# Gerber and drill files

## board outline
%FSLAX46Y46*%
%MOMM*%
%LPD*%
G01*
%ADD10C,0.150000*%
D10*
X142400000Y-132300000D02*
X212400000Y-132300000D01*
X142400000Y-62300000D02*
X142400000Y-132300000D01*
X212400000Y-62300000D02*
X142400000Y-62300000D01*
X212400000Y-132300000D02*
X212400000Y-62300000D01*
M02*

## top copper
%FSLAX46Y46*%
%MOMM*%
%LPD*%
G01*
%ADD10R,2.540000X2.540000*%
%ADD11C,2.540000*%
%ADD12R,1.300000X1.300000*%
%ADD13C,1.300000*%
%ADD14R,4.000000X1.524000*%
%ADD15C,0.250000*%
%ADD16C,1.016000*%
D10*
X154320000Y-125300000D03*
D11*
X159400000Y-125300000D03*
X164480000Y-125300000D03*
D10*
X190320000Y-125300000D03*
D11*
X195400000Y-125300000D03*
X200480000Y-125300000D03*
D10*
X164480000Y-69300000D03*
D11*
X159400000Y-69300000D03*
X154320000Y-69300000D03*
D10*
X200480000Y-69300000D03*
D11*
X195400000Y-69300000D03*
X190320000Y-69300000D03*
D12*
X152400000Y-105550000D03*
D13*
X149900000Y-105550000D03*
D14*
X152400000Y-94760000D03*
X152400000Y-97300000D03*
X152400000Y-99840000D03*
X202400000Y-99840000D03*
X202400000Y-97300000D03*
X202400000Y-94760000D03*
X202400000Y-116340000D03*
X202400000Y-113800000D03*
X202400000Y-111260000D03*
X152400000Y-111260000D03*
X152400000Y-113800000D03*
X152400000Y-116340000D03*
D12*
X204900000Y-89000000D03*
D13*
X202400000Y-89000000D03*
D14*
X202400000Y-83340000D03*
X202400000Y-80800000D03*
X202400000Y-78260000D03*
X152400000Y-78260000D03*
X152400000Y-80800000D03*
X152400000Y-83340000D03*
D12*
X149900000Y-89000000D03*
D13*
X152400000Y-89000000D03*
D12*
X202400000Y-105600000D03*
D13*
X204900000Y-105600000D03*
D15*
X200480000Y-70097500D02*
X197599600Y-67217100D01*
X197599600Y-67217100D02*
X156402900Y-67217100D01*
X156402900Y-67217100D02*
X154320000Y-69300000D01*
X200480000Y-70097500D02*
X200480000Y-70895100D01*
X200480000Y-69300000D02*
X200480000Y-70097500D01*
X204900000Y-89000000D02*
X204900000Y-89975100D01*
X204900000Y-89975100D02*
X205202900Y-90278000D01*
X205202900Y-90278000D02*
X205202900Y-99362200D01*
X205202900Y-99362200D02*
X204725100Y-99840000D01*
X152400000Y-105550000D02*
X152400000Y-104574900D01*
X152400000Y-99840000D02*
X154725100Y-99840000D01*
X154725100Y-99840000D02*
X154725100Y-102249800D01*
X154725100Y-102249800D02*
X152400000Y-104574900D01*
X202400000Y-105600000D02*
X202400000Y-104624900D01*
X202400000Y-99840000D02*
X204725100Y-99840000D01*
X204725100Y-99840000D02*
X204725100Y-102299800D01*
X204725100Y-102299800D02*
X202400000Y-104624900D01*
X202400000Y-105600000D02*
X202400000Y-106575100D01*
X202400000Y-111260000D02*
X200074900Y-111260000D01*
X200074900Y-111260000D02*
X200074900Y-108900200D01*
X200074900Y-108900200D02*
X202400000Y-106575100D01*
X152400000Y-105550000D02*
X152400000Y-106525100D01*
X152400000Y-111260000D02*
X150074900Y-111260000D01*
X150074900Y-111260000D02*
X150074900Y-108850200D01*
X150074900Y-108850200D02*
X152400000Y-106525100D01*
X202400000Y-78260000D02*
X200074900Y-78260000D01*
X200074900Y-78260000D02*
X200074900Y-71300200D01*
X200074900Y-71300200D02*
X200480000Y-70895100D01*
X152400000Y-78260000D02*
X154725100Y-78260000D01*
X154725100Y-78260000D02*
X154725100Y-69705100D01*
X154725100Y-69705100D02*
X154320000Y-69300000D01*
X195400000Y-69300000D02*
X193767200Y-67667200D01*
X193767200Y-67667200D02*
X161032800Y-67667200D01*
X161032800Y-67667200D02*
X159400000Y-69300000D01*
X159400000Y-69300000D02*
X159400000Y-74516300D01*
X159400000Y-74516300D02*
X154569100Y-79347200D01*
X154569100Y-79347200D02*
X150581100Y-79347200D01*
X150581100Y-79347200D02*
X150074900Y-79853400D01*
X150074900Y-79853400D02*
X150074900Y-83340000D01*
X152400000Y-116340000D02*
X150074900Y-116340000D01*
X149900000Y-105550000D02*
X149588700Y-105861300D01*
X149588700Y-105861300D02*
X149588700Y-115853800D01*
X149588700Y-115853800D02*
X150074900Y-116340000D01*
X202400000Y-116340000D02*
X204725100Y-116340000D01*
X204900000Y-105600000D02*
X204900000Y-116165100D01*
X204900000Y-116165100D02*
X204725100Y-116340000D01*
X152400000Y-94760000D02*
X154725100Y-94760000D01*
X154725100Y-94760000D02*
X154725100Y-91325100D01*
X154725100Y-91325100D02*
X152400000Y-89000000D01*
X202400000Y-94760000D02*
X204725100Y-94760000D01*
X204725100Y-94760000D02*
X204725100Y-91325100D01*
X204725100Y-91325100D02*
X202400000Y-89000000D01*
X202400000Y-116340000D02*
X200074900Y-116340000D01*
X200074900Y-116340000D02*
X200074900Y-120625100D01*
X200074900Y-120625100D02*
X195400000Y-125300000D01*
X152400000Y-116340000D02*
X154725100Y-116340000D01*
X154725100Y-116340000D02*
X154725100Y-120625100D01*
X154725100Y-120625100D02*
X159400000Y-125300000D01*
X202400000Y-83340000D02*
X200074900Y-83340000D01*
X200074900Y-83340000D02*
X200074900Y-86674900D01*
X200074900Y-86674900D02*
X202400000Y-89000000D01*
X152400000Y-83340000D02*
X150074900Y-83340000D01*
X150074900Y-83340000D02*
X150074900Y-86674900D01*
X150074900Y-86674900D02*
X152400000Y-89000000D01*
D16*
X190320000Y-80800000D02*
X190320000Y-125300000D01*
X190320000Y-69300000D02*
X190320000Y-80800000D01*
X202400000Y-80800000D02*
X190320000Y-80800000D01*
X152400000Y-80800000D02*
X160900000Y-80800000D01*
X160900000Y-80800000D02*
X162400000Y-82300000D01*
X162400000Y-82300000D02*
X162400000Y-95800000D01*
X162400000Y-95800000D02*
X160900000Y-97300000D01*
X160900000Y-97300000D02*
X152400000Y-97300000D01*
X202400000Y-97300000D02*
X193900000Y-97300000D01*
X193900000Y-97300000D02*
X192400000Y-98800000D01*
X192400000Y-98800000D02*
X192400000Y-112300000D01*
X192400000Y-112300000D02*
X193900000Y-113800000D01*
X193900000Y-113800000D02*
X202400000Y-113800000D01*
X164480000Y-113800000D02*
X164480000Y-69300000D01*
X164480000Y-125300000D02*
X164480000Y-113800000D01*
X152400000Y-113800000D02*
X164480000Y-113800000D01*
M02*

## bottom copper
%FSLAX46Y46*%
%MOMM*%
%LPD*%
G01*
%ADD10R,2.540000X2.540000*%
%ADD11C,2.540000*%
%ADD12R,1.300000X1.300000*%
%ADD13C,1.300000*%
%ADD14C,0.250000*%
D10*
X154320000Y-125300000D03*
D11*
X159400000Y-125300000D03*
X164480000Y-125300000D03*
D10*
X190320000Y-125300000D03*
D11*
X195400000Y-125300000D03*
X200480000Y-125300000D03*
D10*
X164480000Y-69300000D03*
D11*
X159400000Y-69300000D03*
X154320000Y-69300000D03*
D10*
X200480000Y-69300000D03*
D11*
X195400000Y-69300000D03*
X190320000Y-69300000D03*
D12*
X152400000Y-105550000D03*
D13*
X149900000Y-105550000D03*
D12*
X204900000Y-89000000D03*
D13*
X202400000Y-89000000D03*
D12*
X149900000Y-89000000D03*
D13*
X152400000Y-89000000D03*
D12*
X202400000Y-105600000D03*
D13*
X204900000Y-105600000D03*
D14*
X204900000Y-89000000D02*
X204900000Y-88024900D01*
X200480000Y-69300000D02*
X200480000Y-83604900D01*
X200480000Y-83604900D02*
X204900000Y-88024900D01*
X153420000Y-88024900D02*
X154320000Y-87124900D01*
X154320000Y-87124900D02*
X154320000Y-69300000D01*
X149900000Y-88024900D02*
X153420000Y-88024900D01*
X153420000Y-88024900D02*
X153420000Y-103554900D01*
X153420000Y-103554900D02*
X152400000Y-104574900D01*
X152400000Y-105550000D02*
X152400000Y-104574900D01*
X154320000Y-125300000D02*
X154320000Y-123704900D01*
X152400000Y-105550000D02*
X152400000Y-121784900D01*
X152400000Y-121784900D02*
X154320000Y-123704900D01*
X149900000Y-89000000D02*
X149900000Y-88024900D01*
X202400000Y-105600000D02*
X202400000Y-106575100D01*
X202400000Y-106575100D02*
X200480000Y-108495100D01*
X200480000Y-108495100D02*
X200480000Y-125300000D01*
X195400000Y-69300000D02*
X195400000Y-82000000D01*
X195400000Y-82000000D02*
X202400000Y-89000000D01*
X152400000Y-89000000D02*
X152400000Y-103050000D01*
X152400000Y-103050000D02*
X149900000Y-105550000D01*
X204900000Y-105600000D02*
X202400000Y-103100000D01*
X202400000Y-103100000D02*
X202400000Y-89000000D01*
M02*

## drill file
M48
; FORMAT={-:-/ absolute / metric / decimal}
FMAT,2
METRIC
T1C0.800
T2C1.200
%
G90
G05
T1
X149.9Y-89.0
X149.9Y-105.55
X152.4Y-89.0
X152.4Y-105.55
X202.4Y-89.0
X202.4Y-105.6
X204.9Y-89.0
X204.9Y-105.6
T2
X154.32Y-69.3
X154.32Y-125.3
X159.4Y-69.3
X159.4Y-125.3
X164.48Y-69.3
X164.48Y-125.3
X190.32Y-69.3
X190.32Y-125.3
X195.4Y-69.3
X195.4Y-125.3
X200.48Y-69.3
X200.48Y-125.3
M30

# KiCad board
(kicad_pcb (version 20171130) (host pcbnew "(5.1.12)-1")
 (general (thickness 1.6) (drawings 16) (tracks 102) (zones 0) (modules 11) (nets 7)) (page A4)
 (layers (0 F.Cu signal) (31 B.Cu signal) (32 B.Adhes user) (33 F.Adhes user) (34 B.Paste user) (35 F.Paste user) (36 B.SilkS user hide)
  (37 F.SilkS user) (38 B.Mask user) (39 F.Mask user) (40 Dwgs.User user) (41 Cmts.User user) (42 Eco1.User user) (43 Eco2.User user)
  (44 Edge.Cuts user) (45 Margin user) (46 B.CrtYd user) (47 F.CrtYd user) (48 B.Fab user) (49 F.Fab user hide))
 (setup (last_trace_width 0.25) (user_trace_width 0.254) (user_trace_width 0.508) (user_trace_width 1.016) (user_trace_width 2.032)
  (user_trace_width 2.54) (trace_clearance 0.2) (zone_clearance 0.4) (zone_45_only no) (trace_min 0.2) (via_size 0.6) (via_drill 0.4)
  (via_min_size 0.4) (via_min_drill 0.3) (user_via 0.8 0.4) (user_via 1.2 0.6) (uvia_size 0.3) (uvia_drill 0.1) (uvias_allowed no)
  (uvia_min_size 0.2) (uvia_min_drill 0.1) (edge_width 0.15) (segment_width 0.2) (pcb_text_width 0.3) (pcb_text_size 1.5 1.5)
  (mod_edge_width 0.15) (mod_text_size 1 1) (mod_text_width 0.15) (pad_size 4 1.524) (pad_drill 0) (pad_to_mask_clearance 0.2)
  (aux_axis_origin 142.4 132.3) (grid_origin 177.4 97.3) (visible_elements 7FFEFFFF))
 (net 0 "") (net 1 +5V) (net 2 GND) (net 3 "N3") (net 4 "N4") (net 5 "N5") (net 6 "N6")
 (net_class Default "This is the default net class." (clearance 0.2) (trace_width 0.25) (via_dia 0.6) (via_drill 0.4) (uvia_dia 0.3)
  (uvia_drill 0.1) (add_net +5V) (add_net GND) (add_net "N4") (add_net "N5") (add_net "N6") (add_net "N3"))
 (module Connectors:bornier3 (layer F.Cu) (at 159.4 125.3)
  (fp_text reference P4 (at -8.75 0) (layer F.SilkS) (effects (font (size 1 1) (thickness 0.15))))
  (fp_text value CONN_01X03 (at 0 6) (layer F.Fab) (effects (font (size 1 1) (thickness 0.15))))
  (pad 1 thru_hole rect (at -5.08 0) (size 2.54 2.54) (drill 1.2) (layers *.Cu *.Mask) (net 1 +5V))
  (pad 2 thru_hole circle (at 0 0) (size 2.54 2.54) (drill 1.2) (layers *.Cu *.Mask) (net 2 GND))
  (pad 3 thru_hole circle (at 5.08 0) (size 2.54 2.54) (drill 1.2) (layers *.Cu *.Mask) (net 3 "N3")))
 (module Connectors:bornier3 (layer F.Cu) (at 195.4 125.3)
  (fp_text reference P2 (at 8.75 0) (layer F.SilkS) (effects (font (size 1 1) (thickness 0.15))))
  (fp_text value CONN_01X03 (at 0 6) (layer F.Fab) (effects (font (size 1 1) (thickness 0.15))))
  (pad 1 thru_hole rect (at -5.08 0) (size 2.54 2.54) (drill 1.2) (layers *.Cu *.Mask) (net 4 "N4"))
  (pad 2 thru_hole circle (at 0 0) (size 2.54 2.54) (drill 1.2) (layers *.Cu *.Mask) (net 2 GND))
  (pad 3 thru_hole circle (at 5.08 0) (size 2.54 2.54) (drill 1.2) (layers *.Cu *.Mask) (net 1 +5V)))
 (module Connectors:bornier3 (layer F.Cu) (at 159.4 69.3 180)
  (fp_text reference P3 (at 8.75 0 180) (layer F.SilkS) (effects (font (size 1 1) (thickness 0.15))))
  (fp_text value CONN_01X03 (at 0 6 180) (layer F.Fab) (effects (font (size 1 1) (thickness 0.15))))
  (pad 1 thru_hole rect (at -5.08 0 180) (size 2.54 2.54) (drill 1.2) (layers *.Cu *.Mask) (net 3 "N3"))
  (pad 2 thru_hole circle (at 0 0 180) (size 2.54 2.54) (drill 1.2) (layers *.Cu *.Mask) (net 2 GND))
  (pad 3 thru_hole circle (at 5.08 0 180) (size 2.54 2.54) (drill 1.2) (layers *.Cu *.Mask) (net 1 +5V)))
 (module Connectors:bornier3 (layer F.Cu) (at 195.4 69.3 180)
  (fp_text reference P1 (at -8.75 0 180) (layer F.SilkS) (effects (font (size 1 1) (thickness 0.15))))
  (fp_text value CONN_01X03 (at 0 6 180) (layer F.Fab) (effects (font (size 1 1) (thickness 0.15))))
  (pad 1 thru_hole rect (at -5.08 0 180) (size 2.54 2.54) (drill 1.2) (layers *.Cu *.Mask) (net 1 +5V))
  (pad 2 thru_hole circle (at 0 0 180) (size 2.54 2.54) (drill 1.2) (layers *.Cu *.Mask) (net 2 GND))
  (pad 3 thru_hole circle (at 5.08 0 180) (size 2.54 2.54) (drill 1.2) (layers *.Cu *.Mask) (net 4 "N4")))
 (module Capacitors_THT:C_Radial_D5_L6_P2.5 (layer F.Cu) (at 152.4 105.55 180)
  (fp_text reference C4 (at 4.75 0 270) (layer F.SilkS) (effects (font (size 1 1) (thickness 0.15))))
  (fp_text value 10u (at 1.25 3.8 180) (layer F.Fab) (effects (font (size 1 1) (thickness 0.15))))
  (pad 1 thru_hole rect (at 0 0 180) (size 1.3 1.3) (drill 0.8) (layers *.Cu *.Mask) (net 1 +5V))
  (pad 2 thru_hole circle (at 2.5 0 180) (size 1.3 1.3) (drill 0.8) (layers *.Cu *.Mask) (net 2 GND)))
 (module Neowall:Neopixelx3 (layer F.Cu) (at 152.4 97.3)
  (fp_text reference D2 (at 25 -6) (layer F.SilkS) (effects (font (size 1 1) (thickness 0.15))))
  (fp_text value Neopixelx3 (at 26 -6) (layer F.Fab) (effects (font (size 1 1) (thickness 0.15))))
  (pad 1 smd rect (at 0 -2.54) (size 4 1.524) (layers F.Cu F.Paste F.Mask) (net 2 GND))
  (pad 2 smd rect (at 0 0) (size 4 1.524) (layers F.Cu F.Paste F.Mask) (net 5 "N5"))
  (pad 3 smd rect (at 0 2.54) (size 4 1.524) (layers F.Cu F.Paste F.Mask) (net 1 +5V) (thermal_width 0.5) (thermal_gap 0.8))
  (pad 4 smd rect (at 50 2.54) (size 4 1.524) (layers F.Cu F.Paste F.Mask) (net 1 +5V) (thermal_gap 0.8))
  (pad 5 smd rect (at 50 0) (size 4 1.524) (layers F.Cu F.Paste F.Mask) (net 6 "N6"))
  (pad 6 smd rect (at 50 -2.54) (size 4 1.524) (layers F.Cu F.Paste F.Mask) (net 2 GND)))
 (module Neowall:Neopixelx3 (layer F.Cu) (at 202.4 113.8 180)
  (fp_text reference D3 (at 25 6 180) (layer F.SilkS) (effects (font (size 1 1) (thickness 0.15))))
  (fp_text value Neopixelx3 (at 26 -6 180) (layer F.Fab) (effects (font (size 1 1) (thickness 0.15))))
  (pad 1 smd rect (at 0 -2.54 180) (size 4 1.524) (layers F.Cu F.Paste F.Mask) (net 2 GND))
  (pad 2 smd rect (at 0 0 180) (size 4 1.524) (layers F.Cu F.Paste F.Mask) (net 6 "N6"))
  (pad 3 smd rect (at 0 2.54 180) (size 4 1.524) (layers F.Cu F.Paste F.Mask) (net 1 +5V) (thermal_width 0.5) (thermal_gap 0.8))
  (pad 4 smd rect (at 50 2.54 180) (size 4 1.524) (layers F.Cu F.Paste F.Mask) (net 1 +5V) (thermal_width 0.5) (thermal_gap 0.8))
  (pad 5 smd rect (at 50 0 180) (size 4 1.524) (layers F.Cu F.Paste F.Mask) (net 3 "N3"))
  (pad 6 smd rect (at 50 -2.54 180) (size 4 1.524) (layers F.Cu F.Paste F.Mask) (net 2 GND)))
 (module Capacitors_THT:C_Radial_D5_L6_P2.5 (layer F.Cu) (at 204.9 89 180)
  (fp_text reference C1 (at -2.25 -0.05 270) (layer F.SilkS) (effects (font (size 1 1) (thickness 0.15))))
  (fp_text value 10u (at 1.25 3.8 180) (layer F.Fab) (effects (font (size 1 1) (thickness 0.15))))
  (pad 1 thru_hole rect (at 0 0 180) (size 1.3 1.3) (drill 0.8) (layers *.Cu *.Mask) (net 1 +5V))
  (pad 2 thru_hole circle (at 2.5 0 180) (size 1.3 1.3) (drill 0.8) (layers *.Cu *.Mask) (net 2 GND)))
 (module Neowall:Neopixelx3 (layer F.Cu) (at 202.4 80.8 180)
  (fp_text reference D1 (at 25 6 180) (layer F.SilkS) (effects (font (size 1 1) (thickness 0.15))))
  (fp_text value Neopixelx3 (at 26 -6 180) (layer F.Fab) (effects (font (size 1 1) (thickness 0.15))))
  (pad 1 smd rect (at 0 -2.54 180) (size 4 1.524) (layers F.Cu F.Paste F.Mask) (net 2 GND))
  (pad 2 smd rect (at 0 0 180) (size 4 1.524) (layers F.Cu F.Paste F.Mask) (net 4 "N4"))
  (pad 3 smd rect (at 0 2.54 180) (size 4 1.524) (layers F.Cu F.Paste F.Mask) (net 1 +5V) (thermal_width 0.5) (thermal_gap 0.8))
  (pad 4 smd rect (at 50 2.54 180) (size 4 1.524) (layers F.Cu F.Paste F.Mask) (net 1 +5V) (thermal_width 0.5) (thermal_gap 0.8))
  (pad 5 smd rect (at 50 0 180) (size 4 1.524) (layers F.Cu F.Paste F.Mask) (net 5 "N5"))
  (pad 6 smd rect (at 50 -2.54 180) (size 4 1.524) (layers F.Cu F.Paste F.Mask) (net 2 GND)))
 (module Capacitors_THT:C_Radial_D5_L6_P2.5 (layer F.Cu) (at 149.9 89)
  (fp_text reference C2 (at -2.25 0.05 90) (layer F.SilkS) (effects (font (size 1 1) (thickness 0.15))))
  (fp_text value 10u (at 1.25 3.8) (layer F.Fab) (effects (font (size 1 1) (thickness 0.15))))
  (pad 1 thru_hole rect (at 0 0) (size 1.3 1.3) (drill 0.8) (layers *.Cu *.Mask) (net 1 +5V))
  (pad 2 thru_hole circle (at 2.5 0) (size 1.3 1.3) (drill 0.8) (layers *.Cu *.Mask) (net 2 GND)))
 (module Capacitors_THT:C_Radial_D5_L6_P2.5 (layer F.Cu) (at 202.4 105.6)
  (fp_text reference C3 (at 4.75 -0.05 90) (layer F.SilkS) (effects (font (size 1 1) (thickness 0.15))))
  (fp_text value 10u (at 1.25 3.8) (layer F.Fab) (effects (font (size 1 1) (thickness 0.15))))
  (pad 1 thru_hole rect (at 0 0) (size 1.3 1.3) (drill 0.8) (layers *.Cu *.Mask) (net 1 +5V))
  (pad 2 thru_hole circle (at 2.5 0) (size 1.3 1.3) (drill 0.8) (layers *.Cu *.Mask) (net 2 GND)))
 (gr_line (start 142.4 132.3) (end 212.4 132.3) (angle 90) (layer Edge.Cuts) (width 0.15))
 (gr_line (start 142.4 62.3) (end 142.4 132.3) (angle 90) (layer Edge.Cuts) (width 0.15))
 (gr_line (start 212.4 62.3) (end 142.4 62.3) (angle 90) (layer Edge.Cuts) (width 0.15))
 (gr_line (start 212.4 132.3) (end 212.4 62.3) (angle 90) (layer Edge.Cuts) (width 0.15))
 (segment (start 200.48 70.0975) (end 197.5996 67.2171) (width 0.25) (layer F.Cu) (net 1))
 (segment (start 197.5996 67.2171) (end 156.4029 67.2171) (width 0.25) (layer F.Cu) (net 1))
 (segment (start 156.4029 67.2171) (end 154.32 69.3) (width 0.25) (layer F.Cu) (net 1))
 (segment (start 200.48 70.0975) (end 200.48 70.8951) (width 0.25) (layer F.Cu) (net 1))
 (segment (start 200.48 69.3) (end 200.48 70.0975) (width 0.25) (layer F.Cu) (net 1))
 (segment (start 204.9 89) (end 204.9 88.0249) (width 0.25) (layer B.Cu) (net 1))
 (segment (start 200.48 69.3) (end 200.48 83.6049) (width 0.25) (layer B.Cu) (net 1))
 (segment (start 200.48 83.6049) (end 204.9 88.0249) (width 0.25) (layer B.Cu) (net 1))
 (segment (start 153.42 88.0249) (end 154.32 87.1249) (width 0.25) (layer B.Cu) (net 1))
 (segment (start 154.32 87.1249) (end 154.32 69.3) (width 0.25) (layer B.Cu) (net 1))
 (segment (start 149.9 88.0249) (end 153.42 88.0249) (width 0.25) (layer B.Cu) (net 1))
 (segment (start 153.42 88.0249) (end 153.42 103.5549) (width 0.25) (layer B.Cu) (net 1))
 (segment (start 153.42 103.5549) (end 152.4 104.5749) (width 0.25) (layer B.Cu) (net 1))
 (segment (start 152.4 105.55) (end 152.4 104.5749) (width 0.25) (layer B.Cu) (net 1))
 (segment (start 154.32 125.3) (end 154.32 123.7049) (width 0.25) (layer B.Cu) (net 1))
 (segment (start 152.4 105.55) (end 152.4 121.7849) (width 0.25) (layer B.Cu) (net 1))
 (segment (start 152.4 121.7849) (end 154.32 123.7049) (width 0.25) (layer B.Cu) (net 1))
 (segment (start 204.9 89) (end 204.9 89.9751) (width 0.25) (layer F.Cu) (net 1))
 (segment (start 204.9 89.9751) (end 205.2029 90.278) (width 0.25) (layer F.Cu) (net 1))
 (segment (start 205.2029 90.278) (end 205.2029 99.3622) (width 0.25) (layer F.Cu) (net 1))
 (segment (start 205.2029 99.3622) (end 204.7251 99.84) (width 0.25) (layer F.Cu) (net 1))
 (segment (start 149.9 89) (end 149.9 88.0249) (width 0.25) (layer B.Cu) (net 1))
 (segment (start 202.4 105.6) (end 202.4 106.5751) (width 0.25) (layer B.Cu) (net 1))
 (segment (start 202.4 106.5751) (end 200.48 108.4951) (width 0.25) (layer B.Cu) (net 1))
 (segment (start 200.48 108.4951) (end 200.48 125.3) (width 0.25) (layer B.Cu) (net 1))
 (segment (start 152.4 105.55) (end 152.4 104.5749) (width 0.25) (layer F.Cu) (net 1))
 (segment (start 152.4 99.84) (end 154.7251 99.84) (width 0.25) (layer F.Cu) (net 1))
 (segment (start 154.7251 99.84) (end 154.7251 102.2498) (width 0.25) (layer F.Cu) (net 1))
 (segment (start 154.7251 102.2498) (end 152.4 104.5749) (width 0.25) (layer F.Cu) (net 1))
 (segment (start 202.4 105.6) (end 202.4 104.6249) (width 0.25) (layer F.Cu) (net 1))
 (segment (start 202.4 99.84) (end 204.7251 99.84) (width 0.25) (layer F.Cu) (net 1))
 (segment (start 204.7251 99.84) (end 204.7251 102.2998) (width 0.25) (layer F.Cu) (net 1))
 (segment (start 204.7251 102.2998) (end 202.4 104.6249) (width 0.25) (layer F.Cu) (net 1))
 (segment (start 202.4 105.6) (end 202.4 106.5751) (width 0.25) (layer F.Cu) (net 1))
 (segment (start 202.4 111.26) (end 200.0749 111.26) (width 0.25) (layer F.Cu) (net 1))
 (segment (start 200.0749 111.26) (end 200.0749 108.9002) (width 0.25) (layer F.Cu) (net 1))
 (segment (start 200.0749 108.9002) (end 202.4 106.5751) (width 0.25) (layer F.Cu) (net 1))
 (segment (start 152.4 105.55) (end 152.4 106.5251) (width 0.25) (layer F.Cu) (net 1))
 (segment (start 152.4 111.26) (end 150.0749 111.26) (width 0.25) (layer F.Cu) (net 1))
 (segment (start 150.0749 111.26) (end 150.0749 108.8502) (width 0.25) (layer F.Cu) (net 1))
 (segment (start 150.0749 108.8502) (end 152.4 106.5251) (width 0.25) (layer F.Cu) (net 1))
 (segment (start 202.4 78.26) (end 200.0749 78.26) (width 0.25) (layer F.Cu) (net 1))
 (segment (start 200.0749 78.26) (end 200.0749 71.3002) (width 0.25) (layer F.Cu) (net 1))
 (segment (start 200.0749 71.3002) (end 200.48 70.8951) (width 0.25) (layer F.Cu) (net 1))
 (segment (start 152.4 78.26) (end 154.7251 78.26) (width 0.25) (layer F.Cu) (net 1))
 (segment (start 154.7251 78.26) (end 154.7251 69.7051) (width 0.25) (layer F.Cu) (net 1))
 (segment (start 154.7251 69.7051) (end 154.32 69.3) (width 0.25) (layer F.Cu) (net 1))
 (segment (start 195.4 69.3) (end 193.7672 67.6672) (width 0.25) (layer F.Cu) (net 2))
 (segment (start 193.7672 67.6672) (end 161.0328 67.6672) (width 0.25) (layer F.Cu) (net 2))
 (segment (start 161.0328 67.6672) (end 159.4 69.3) (width 0.25) (layer F.Cu) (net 2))
 (segment (start 195.4 69.3) (end 195.4 82) (width 0.25) (layer B.Cu) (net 2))
 (segment (start 195.4 82) (end 202.4 89) (width 0.25) (layer B.Cu) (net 2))
 (segment (start 159.4 69.3) (end 159.4 74.5163) (width 0.25) (layer F.Cu) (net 2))
 (segment (start 159.4 74.5163) (end 154.5691 79.3472) (width 0.25) (layer F.Cu) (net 2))
 (segment (start 154.5691 79.3472) (end 150.5811 79.3472) (width 0.25) (layer F.Cu) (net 2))
 (segment (start 150.5811 79.3472) (end 150.0749 79.8534) (width 0.25) (layer F.Cu) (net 2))
 (segment (start 150.0749 79.8534) (end 150.0749 83.34) (width 0.25) (layer F.Cu) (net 2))
 (segment (start 152.4 89) (end 152.4 103.05) (width 0.25) (layer B.Cu) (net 2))
 (segment (start 152.4 103.05) (end 149.9 105.55) (width 0.25) (layer B.Cu) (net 2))
 (segment (start 152.4 116.34) (end 150.0749 116.34) (width 0.25) (layer F.Cu) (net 2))
 (segment (start 149.9 105.55) (end 149.5887 105.8613) (width 0.25) (layer F.Cu) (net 2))
 (segment (start 149.5887 105.8613) (end 149.5887 115.8538) (width 0.25) (layer F.Cu) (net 2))
 (segment (start 149.5887 115.8538) (end 150.0749 116.34) (width 0.25) (layer F.Cu) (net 2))
 (segment (start 202.4 116.34) (end 204.7251 116.34) (width 0.25) (layer F.Cu) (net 2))
 (segment (start 204.9 105.6) (end 204.9 116.1651) (width 0.25) (layer F.Cu) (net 2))
 (segment (start 204.9 116.1651) (end 204.7251 116.34) (width 0.25) (layer F.Cu) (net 2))
 (segment (start 204.9 105.6) (end 202.4 103.1) (width 0.25) (layer B.Cu) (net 2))
 (segment (start 202.4 103.1) (end 202.4 89) (width 0.25) (layer B.Cu) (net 2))
 (segment (start 152.4 94.76) (end 154.7251 94.76) (width 0.25) (layer F.Cu) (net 2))
 (segment (start 154.7251 94.76) (end 154.7251 91.3251) (width 0.25) (layer F.Cu) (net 2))
 (segment (start 154.7251 91.3251) (end 152.4 89) (width 0.25) (layer F.Cu) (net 2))
 (segment (start 202.4 94.76) (end 204.7251 94.76) (width 0.25) (layer F.Cu) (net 2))
 (segment (start 204.7251 94.76) (end 204.7251 91.3251) (width 0.25) (layer F.Cu) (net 2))
 (segment (start 204.7251 91.3251) (end 202.4 89) (width 0.25) (layer F.Cu) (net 2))
 (segment (start 202.4 116.34) (end 200.0749 116.34) (width 0.25) (layer F.Cu) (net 2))
 (segment (start 200.0749 116.34) (end 200.0749 120.6251) (width 0.25) (layer F.Cu) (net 2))
 (segment (start 200.0749 120.6251) (end 195.4 125.3) (width 0.25) (layer F.Cu) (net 2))
 (segment (start 152.4 116.34) (end 154.7251 116.34) (width 0.25) (layer F.Cu) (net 2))
 (segment (start 154.7251 116.34) (end 154.7251 120.6251) (width 0.25) (layer F.Cu) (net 2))
 (segment (start 154.7251 120.6251) (end 159.4 125.3) (width 0.25) (layer F.Cu) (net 2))
 (segment (start 202.4 83.34) (end 200.0749 83.34) (width 0.25) (layer F.Cu) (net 2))
 (segment (start 200.0749 83.34) (end 200.0749 86.6749) (width 0.25) (layer F.Cu) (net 2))
 (segment (start 200.0749 86.6749) (end 202.4 89) (width 0.25) (layer F.Cu) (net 2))
 (segment (start 152.4 83.34) (end 150.0749 83.34) (width 0.25) (layer F.Cu) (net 2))
 (segment (start 150.0749 83.34) (end 150.0749 86.6749) (width 0.25) (layer F.Cu) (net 2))
 (segment (start 150.0749 86.6749) (end 152.4 89) (width 0.25) (layer F.Cu) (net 2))
 (segment (start 190.32 80.8) (end 190.32 125.3) (width 1.016) (layer F.Cu) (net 4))
 (segment (start 190.32 69.3) (end 190.32 80.8) (width 1.016) (layer F.Cu) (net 4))
 (segment (start 202.4 80.8) (end 190.32 80.8) (width 1.016) (layer F.Cu) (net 4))
 (segment (start 152.4 80.8) (end 160.9 80.8) (width 1.016) (layer F.Cu) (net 5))
 (segment (start 160.9 80.8) (end 162.4 82.3) (width 1.016) (layer F.Cu) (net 5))
 (segment (start 162.4 82.3) (end 162.4 95.8) (width 1.016) (layer F.Cu) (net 5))
 (segment (start 162.4 95.8) (end 160.9 97.3) (width 1.016) (layer F.Cu) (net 5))
 (segment (start 160.9 97.3) (end 152.4 97.3) (width 1.016) (layer F.Cu) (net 5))
 (segment (start 202.4 97.3) (end 193.9 97.3) (width 1.016) (layer F.Cu) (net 6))
 (segment (start 193.9 97.3) (end 192.4 98.8) (width 1.016) (layer F.Cu) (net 6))
 (segment (start 192.4 98.8) (end 192.4 112.3) (width 1.016) (layer F.Cu) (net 6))
 (segment (start 192.4 112.3) (end 193.9 113.8) (width 1.016) (layer F.Cu) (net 6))
 (segment (start 193.9 113.8) (end 202.4 113.8) (width 1.016) (layer F.Cu) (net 6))
 (segment (start 164.48 113.8) (end 164.48 69.3) (width 1.016) (layer F.Cu) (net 3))
 (segment (start 164.48 125.3) (end 164.48 113.8) (width 1.016) (layer F.Cu) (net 3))
 (segment (start 152.4 113.8) (end 164.48 113.8) (width 1.016) (layer F.Cu) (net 3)))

